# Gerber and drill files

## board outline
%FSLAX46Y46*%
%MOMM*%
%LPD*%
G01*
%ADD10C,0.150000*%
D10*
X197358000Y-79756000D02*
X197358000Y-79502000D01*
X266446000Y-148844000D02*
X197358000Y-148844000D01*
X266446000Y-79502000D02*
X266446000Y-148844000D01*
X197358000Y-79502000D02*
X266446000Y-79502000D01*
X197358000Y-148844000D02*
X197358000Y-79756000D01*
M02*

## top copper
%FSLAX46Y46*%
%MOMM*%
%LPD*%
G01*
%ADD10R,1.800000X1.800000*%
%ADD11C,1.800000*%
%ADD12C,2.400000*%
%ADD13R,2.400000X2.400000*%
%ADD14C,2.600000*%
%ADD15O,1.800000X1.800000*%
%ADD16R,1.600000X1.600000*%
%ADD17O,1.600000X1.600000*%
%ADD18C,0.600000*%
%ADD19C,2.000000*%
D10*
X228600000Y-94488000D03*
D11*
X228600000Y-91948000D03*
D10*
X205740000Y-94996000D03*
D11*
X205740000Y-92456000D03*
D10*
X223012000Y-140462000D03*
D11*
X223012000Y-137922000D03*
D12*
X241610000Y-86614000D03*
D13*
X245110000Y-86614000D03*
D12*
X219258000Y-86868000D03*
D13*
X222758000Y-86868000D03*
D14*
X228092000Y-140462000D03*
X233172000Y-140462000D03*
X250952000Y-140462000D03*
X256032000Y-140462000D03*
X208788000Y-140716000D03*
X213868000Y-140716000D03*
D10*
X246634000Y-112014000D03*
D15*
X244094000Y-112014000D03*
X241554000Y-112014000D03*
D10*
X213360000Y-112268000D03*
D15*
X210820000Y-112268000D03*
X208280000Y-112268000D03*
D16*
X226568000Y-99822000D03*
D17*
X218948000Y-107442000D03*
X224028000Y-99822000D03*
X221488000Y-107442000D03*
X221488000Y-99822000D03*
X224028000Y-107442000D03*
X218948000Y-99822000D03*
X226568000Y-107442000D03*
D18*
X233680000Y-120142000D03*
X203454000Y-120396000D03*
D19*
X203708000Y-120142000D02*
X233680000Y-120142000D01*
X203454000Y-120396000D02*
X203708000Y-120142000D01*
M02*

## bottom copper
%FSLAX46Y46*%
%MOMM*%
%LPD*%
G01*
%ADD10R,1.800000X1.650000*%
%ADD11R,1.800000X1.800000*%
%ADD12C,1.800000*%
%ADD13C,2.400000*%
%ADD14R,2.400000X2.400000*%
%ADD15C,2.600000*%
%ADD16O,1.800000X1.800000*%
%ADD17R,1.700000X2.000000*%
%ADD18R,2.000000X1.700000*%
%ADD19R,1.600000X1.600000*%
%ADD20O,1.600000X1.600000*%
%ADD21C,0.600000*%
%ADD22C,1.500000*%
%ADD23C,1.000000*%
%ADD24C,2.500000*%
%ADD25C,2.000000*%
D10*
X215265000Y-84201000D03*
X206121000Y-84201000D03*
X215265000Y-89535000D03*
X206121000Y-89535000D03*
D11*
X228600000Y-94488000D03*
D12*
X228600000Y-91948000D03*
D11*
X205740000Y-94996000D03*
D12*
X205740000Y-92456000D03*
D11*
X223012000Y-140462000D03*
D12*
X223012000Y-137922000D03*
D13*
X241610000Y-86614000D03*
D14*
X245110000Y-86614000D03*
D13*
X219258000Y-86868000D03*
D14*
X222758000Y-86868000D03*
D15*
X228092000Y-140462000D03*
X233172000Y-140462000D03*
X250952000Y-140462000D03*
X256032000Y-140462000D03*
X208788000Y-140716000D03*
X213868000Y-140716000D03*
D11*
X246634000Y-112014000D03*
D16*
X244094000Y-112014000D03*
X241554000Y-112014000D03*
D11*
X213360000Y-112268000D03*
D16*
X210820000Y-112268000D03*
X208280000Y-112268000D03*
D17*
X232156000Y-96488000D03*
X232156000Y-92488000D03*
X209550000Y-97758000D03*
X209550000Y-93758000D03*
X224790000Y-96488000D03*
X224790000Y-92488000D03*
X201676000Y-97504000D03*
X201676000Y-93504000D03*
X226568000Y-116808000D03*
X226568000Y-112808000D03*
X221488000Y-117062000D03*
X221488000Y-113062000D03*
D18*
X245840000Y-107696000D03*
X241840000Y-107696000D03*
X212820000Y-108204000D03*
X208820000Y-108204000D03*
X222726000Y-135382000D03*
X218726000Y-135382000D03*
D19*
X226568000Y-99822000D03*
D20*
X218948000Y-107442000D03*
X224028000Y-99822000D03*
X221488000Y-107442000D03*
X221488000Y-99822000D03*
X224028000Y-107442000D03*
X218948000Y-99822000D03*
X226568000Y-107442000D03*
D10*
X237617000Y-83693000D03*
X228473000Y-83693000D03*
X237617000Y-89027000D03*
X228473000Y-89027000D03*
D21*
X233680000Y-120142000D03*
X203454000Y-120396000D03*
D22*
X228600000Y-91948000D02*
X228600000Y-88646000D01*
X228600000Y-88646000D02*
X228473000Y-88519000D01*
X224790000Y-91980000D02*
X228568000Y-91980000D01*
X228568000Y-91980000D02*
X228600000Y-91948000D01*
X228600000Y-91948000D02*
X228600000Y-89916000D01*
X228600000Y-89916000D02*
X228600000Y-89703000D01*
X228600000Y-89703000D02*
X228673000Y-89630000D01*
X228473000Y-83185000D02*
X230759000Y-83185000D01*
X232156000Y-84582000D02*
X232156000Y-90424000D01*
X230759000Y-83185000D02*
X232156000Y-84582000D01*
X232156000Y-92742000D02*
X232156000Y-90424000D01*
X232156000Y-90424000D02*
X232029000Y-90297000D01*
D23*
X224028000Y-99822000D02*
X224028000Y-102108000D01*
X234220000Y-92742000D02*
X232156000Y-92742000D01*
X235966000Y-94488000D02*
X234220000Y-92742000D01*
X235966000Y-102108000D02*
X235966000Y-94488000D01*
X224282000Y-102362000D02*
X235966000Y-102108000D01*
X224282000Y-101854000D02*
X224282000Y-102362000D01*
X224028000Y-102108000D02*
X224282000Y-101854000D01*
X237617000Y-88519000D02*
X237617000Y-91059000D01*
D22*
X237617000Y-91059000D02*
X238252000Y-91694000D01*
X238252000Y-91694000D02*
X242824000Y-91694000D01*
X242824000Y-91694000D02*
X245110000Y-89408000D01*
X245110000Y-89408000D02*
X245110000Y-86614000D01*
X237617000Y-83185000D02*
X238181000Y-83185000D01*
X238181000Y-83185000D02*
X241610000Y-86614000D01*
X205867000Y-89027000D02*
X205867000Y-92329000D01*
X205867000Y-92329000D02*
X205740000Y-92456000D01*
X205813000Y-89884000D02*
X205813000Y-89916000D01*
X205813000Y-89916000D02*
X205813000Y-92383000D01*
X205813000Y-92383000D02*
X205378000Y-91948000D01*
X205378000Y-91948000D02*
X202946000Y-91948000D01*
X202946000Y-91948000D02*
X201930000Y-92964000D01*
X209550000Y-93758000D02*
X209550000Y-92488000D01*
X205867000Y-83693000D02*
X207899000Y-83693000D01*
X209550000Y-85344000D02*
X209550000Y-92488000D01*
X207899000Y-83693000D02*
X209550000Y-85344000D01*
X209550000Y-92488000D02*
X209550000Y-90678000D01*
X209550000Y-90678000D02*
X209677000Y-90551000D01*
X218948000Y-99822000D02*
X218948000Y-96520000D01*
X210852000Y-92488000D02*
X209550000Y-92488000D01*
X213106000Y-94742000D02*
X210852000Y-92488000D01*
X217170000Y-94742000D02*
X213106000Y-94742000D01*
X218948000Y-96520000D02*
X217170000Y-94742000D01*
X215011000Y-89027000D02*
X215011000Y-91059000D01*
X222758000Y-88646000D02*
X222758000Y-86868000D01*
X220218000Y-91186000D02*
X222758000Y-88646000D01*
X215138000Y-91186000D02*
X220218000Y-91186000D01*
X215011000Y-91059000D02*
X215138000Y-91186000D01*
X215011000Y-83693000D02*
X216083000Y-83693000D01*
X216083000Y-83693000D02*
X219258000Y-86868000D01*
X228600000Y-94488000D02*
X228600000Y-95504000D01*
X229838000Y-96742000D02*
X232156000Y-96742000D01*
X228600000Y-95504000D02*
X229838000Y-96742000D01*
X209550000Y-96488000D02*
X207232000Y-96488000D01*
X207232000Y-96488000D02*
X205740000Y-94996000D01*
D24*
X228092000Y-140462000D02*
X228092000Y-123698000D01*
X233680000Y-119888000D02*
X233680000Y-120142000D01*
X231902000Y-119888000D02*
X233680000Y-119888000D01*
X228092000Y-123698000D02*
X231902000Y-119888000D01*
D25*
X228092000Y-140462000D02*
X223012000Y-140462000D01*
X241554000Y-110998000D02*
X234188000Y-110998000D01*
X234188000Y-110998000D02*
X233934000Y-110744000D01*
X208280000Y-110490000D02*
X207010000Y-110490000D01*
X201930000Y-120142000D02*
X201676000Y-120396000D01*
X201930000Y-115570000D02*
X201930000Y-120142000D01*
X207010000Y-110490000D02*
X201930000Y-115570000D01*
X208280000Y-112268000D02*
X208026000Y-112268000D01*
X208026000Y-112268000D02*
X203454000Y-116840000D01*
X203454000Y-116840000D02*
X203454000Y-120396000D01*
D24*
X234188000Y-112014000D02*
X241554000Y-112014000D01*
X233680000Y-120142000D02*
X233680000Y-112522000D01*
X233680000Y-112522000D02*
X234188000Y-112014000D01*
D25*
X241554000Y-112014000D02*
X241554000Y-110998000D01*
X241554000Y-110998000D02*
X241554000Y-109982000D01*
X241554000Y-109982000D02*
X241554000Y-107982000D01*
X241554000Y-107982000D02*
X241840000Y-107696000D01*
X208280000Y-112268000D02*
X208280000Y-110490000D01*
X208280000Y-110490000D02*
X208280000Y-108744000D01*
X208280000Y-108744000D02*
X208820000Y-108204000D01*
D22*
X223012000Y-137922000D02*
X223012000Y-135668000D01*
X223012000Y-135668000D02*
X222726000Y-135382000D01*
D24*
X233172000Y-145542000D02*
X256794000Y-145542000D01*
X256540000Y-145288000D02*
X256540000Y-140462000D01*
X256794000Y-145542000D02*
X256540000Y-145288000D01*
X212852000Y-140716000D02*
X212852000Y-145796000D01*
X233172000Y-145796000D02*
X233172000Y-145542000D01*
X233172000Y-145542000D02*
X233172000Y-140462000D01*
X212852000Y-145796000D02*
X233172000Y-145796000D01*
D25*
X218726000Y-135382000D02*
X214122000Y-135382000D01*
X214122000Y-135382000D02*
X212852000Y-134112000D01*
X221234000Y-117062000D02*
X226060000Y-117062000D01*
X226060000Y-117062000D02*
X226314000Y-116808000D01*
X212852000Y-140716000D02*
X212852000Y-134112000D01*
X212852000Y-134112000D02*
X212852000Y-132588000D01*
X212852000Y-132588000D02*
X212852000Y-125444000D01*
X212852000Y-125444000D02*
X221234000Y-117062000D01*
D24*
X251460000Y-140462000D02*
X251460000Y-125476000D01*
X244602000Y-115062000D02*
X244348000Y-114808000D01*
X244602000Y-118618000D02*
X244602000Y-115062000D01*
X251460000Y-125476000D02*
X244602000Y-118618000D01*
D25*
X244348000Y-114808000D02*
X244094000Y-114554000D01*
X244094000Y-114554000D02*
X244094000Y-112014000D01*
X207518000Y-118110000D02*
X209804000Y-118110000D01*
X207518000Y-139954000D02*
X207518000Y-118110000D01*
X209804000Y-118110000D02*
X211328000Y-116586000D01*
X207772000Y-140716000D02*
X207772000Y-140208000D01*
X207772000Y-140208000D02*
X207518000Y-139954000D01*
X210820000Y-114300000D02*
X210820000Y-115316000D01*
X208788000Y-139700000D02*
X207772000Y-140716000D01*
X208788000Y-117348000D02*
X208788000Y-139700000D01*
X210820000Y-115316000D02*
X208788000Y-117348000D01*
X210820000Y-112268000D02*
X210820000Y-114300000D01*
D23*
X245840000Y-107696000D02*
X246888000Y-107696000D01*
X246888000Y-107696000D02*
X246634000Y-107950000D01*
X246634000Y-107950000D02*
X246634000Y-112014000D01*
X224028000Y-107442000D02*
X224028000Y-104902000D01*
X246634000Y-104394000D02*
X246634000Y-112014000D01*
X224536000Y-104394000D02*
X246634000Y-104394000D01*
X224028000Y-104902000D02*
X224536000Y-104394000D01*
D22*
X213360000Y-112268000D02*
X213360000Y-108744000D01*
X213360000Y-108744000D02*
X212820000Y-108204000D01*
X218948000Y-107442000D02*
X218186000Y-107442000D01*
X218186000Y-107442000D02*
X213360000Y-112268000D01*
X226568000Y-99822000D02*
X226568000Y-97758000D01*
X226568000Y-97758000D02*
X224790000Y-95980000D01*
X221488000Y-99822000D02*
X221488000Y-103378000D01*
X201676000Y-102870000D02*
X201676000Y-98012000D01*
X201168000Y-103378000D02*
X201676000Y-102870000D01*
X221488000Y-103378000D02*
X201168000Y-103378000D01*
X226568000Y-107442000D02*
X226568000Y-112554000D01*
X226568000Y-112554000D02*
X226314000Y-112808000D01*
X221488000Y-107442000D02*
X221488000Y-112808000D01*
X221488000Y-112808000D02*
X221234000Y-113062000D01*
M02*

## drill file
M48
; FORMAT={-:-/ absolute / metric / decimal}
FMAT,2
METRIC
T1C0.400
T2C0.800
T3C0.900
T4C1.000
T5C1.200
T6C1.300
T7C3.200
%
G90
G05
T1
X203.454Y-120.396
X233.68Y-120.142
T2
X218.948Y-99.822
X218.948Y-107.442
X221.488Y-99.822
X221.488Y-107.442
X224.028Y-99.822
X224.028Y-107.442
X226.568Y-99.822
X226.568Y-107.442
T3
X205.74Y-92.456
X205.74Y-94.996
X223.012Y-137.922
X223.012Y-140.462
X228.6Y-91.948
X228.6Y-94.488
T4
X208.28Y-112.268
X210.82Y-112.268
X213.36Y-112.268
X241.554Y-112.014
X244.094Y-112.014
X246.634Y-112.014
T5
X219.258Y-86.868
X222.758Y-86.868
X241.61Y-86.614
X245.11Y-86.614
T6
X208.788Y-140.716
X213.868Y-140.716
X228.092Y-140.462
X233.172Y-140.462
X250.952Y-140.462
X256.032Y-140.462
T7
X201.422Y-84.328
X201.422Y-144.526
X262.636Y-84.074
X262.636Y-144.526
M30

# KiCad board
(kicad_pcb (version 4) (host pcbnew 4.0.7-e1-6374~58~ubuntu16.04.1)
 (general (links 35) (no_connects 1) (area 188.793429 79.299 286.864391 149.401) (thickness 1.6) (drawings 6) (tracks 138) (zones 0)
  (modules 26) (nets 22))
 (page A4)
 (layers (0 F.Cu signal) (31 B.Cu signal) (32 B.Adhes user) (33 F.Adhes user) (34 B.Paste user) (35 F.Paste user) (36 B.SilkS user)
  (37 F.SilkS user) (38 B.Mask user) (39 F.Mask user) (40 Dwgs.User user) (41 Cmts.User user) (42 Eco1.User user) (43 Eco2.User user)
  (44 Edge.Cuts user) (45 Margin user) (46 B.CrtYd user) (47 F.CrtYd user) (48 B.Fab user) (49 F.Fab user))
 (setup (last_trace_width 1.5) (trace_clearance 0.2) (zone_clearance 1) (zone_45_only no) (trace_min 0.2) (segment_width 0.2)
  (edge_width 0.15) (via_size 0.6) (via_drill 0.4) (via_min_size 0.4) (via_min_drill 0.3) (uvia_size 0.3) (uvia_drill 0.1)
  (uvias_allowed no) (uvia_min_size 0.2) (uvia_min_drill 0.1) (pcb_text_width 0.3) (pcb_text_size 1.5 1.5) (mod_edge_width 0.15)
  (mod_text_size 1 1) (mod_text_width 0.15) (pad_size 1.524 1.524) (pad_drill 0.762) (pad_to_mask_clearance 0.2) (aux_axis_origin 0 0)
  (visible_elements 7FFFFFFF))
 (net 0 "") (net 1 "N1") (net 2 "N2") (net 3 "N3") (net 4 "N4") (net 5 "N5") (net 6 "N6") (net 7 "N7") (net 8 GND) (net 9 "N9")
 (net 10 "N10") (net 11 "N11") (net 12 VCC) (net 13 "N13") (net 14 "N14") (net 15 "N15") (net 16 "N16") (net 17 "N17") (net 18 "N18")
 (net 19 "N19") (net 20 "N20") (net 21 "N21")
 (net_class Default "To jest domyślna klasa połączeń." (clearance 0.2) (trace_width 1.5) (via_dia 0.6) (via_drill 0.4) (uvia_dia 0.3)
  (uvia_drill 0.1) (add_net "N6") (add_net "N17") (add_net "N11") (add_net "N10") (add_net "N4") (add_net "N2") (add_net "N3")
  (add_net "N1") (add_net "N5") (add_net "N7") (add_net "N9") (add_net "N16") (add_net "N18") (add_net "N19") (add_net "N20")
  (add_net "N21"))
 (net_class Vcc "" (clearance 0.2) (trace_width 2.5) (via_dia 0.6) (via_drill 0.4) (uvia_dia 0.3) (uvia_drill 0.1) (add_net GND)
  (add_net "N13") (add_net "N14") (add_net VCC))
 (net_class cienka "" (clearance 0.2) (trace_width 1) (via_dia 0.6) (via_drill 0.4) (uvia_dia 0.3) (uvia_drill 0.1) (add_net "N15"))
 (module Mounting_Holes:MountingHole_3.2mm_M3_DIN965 (layer F.Cu) (at 262.636 144.526)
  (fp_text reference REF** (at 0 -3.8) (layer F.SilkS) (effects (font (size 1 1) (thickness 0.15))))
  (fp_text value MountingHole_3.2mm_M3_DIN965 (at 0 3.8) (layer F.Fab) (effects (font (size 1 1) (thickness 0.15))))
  (pad 1 np_thru_hole circle (at 0 0) (size 3.2 3.2) (drill 3.2) (layers *.Cu *.Mask)))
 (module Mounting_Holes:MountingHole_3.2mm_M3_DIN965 (layer F.Cu) (at 201.422 144.526)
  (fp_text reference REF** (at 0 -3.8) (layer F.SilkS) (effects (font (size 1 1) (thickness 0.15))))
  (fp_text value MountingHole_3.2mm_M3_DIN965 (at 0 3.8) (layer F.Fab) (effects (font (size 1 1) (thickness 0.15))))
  (pad 1 np_thru_hole circle (at 0 0) (size 3.2 3.2) (drill 3.2) (layers *.Cu *.Mask)))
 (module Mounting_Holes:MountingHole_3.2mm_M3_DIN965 (layer F.Cu) (at 201.422 84.328)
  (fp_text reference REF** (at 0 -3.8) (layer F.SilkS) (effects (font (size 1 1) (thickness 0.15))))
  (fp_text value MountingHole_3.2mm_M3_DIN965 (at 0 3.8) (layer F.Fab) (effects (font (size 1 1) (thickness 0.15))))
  (pad 1 np_thru_hole circle (at 0 0) (size 3.2 3.2) (drill 3.2) (layers *.Cu *.Mask)))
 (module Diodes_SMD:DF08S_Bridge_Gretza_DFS (layer B.Cu) (at 210.566 86.868 270)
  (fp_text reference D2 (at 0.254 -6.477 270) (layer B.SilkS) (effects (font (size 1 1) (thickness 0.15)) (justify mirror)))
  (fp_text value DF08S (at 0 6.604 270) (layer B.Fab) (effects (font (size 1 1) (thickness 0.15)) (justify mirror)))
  (pad 4 smd rect (at -2.667 -4.699 270) (size 1.65 1.8) (layers B.Cu B.Paste B.Mask) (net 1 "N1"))
  (pad 2 smd rect (at -2.667 4.445 270) (size 1.65 1.8) (layers B.Cu B.Paste B.Mask) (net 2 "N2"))
  (pad 3 smd rect (at 2.667 -4.699 270) (size 1.65 1.8) (layers B.Cu B.Paste B.Mask) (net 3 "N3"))
  (pad 1 smd rect (at 2.667 4.445 270) (size 1.65 1.8) (layers B.Cu B.Paste B.Mask) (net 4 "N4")))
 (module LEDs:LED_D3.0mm (layer F.Cu) (at 228.6 94.488 90)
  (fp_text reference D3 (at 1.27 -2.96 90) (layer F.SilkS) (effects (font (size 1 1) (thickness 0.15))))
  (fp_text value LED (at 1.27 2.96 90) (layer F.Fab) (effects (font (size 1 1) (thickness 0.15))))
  (pad 1 thru_hole rect (at 0 0 90) (size 1.8 1.8) (drill 0.9) (layers *.Cu *.Mask) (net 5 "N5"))
  (pad 2 thru_hole circle (at 2.54 0 90) (size 1.8 1.8) (drill 0.9) (layers *.Cu *.Mask) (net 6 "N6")))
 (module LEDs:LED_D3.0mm (layer F.Cu) (at 205.74 94.996 90)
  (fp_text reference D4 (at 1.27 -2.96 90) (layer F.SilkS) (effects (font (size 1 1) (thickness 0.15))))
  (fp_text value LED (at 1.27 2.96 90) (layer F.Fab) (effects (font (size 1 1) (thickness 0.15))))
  (pad 1 thru_hole rect (at 0 0 90) (size 1.8 1.8) (drill 0.9) (layers *.Cu *.Mask) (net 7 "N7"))
  (pad 2 thru_hole circle (at 2.54 0 90) (size 1.8 1.8) (drill 0.9) (layers *.Cu *.Mask) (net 4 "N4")))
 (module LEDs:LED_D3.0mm (layer F.Cu) (at 223.012 140.462 90)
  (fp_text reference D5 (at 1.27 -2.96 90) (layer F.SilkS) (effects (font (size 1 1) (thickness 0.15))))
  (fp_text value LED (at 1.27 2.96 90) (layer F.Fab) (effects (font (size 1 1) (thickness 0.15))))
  (pad 1 thru_hole rect (at 0 0 90) (size 1.8 1.8) (drill 0.9) (layers *.Cu *.Mask) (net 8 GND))
  (pad 2 thru_hole circle (at 2.54 0 90) (size 1.8 1.8) (drill 0.9) (layers *.Cu *.Mask) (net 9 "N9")))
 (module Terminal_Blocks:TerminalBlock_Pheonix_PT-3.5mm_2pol (layer F.Cu) (at 245.11 86.614 180)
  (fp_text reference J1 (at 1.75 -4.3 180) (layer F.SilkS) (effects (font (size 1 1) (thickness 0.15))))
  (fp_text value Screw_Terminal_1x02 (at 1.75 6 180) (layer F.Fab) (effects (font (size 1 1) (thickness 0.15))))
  (pad 2 thru_hole circle (at 3.5 0 180) (size 2.4 2.4) (drill 1.2) (layers *.Cu *.Mask F.SilkS) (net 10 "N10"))
  (pad 1 thru_hole rect (at 0 0 180) (size 2.4 2.4) (drill 1.2) (layers *.Cu *.Mask F.SilkS) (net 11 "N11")))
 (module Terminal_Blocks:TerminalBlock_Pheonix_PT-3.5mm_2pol (layer F.Cu) (at 222.758 86.868 180)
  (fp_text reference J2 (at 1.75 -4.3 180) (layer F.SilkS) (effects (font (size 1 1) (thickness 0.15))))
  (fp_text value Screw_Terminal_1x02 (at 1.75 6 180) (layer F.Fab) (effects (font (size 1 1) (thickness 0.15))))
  (pad 2 thru_hole circle (at 3.5 0 180) (size 2.4 2.4) (drill 1.2) (layers *.Cu *.Mask F.SilkS) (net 1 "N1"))
  (pad 1 thru_hole rect (at 0 0 180) (size 2.4 2.4) (drill 1.2) (layers *.Cu *.Mask F.SilkS) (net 3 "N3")))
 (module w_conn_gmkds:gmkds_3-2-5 (layer F.Cu) (at 230.632 140.462)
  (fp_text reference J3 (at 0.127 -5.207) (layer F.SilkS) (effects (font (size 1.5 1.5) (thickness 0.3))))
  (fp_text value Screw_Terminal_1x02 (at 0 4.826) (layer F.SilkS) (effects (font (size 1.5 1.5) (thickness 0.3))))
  (pad 1 thru_hole circle (at -2.54 0) (size 2.6 2.6) (drill 1.3) (layers *.Cu *.Mask F.SilkS) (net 8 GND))
  (pad 2 thru_hole circle (at 2.54 0) (size 2.6 2.6) (drill 1.3) (layers *.Cu *.Mask F.SilkS) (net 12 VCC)))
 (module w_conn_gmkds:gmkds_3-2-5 (layer F.Cu) (at 253.492 140.462)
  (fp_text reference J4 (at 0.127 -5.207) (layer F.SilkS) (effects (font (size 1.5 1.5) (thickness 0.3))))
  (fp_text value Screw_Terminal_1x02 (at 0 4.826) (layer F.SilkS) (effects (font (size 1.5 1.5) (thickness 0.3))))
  (pad 1 thru_hole circle (at -2.54 0) (size 2.6 2.6) (drill 1.3) (layers *.Cu *.Mask F.SilkS) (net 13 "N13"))
  (pad 2 thru_hole circle (at 2.54 0) (size 2.6 2.6) (drill 1.3) (layers *.Cu *.Mask F.SilkS) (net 12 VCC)))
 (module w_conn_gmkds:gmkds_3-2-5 (layer F.Cu) (at 211.328 140.716)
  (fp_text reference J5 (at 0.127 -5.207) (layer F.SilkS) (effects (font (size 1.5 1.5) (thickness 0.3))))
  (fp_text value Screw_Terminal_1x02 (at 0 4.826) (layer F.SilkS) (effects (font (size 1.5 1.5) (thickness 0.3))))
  (pad 1 thru_hole circle (at -2.54 0) (size 2.6 2.6) (drill 1.3) (layers *.Cu *.Mask F.SilkS) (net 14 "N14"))
  (pad 2 thru_hole circle (at 2.54 0) (size 2.6 2.6) (drill 1.3) (layers *.Cu *.Mask F.SilkS) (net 12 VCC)))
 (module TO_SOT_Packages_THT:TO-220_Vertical (layer F.Cu) (at 246.634 112.014 180)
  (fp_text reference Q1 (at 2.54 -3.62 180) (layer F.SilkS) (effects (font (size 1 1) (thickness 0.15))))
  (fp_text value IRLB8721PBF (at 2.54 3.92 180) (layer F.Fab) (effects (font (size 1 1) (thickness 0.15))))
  (pad 1 thru_hole rect (at 0 0 180) (size 1.8 1.8) (drill 1) (layers *.Cu *.Mask) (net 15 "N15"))
  (pad 2 thru_hole oval (at 2.54 0 180) (size 1.8 1.8) (drill 1) (layers *.Cu *.Mask) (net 13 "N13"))
  (pad 3 thru_hole oval (at 5.08 0 180) (size 1.8 1.8) (drill 1) (layers *.Cu *.Mask) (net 8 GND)))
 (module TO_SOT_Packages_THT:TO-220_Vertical (layer F.Cu) (at 213.36 112.268 180)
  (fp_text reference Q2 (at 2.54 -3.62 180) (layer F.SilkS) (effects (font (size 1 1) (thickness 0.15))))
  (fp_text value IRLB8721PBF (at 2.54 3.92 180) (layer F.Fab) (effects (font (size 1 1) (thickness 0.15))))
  (pad 1 thru_hole rect (at 0 0 180) (size 1.8 1.8) (drill 1) (layers *.Cu *.Mask) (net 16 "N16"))
  (pad 2 thru_hole oval (at 2.54 0 180) (size 1.8 1.8) (drill 1) (layers *.Cu *.Mask) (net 14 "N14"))
  (pad 3 thru_hole oval (at 5.08 0 180) (size 1.8 1.8) (drill 1) (layers *.Cu *.Mask) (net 8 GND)))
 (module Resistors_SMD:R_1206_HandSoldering (layer B.Cu) (at 232.156 94.488 90)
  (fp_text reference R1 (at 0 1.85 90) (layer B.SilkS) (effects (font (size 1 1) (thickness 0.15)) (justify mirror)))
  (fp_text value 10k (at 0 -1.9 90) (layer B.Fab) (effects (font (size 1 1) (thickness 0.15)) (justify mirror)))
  (pad 1 smd rect (at -2 0 90) (size 2 1.7) (layers B.Cu B.Paste B.Mask) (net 5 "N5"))
  (pad 2 smd rect (at 2 0 90) (size 2 1.7) (layers B.Cu B.Paste B.Mask) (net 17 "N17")))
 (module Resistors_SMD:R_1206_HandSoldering (layer B.Cu) (at 209.55 95.758 90)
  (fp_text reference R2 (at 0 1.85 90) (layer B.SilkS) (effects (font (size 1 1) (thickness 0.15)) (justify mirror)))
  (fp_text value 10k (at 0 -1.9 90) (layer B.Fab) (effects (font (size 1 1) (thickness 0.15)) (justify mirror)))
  (pad 1 smd rect (at -2 0 90) (size 2 1.7) (layers B.Cu B.Paste B.Mask) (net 7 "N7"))
  (pad 2 smd rect (at 2 0 90) (size 2 1.7) (layers B.Cu B.Paste B.Mask) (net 2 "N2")))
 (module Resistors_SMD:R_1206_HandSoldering (layer B.Cu) (at 224.79 94.488 90)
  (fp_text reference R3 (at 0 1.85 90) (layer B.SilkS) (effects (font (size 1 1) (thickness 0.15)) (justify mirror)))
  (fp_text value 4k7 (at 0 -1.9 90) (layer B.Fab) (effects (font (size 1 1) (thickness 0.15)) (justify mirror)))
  (pad 1 smd rect (at -2 0 90) (size 2 1.7) (layers B.Cu B.Paste B.Mask) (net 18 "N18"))
  (pad 2 smd rect (at 2 0 90) (size 2 1.7) (layers B.Cu B.Paste B.Mask) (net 6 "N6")))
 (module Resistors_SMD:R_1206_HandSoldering (layer B.Cu) (at 201.676 95.504 90)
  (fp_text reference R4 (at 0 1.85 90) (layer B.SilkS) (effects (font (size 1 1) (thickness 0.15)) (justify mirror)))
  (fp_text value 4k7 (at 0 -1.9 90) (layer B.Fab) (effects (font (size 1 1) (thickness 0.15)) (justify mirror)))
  (pad 1 smd rect (at -2 0 90) (size 2 1.7) (layers B.Cu B.Paste B.Mask) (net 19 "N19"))
  (pad 2 smd rect (at 2 0 90) (size 2 1.7) (layers B.Cu B.Paste B.Mask) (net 4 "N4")))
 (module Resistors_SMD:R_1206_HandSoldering (layer B.Cu) (at 226.568 114.808 90)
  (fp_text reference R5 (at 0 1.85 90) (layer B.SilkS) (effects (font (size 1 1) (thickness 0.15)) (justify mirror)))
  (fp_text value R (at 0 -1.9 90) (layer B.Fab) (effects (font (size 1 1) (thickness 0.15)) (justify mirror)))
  (pad 1 smd rect (at -2 0 90) (size 2 1.7) (layers B.Cu B.Paste B.Mask) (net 12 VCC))
  (pad 2 smd rect (at 2 0 90) (size 2 1.7) (layers B.Cu B.Paste B.Mask) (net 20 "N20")))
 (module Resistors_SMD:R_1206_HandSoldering (layer B.Cu) (at 221.488 115.062 90)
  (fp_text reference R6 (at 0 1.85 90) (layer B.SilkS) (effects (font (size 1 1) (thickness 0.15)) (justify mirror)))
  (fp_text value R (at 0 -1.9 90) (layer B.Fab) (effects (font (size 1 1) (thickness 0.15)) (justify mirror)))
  (pad 1 smd rect (at -2 0 90) (size 2 1.7) (layers B.Cu B.Paste B.Mask) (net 12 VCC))
  (pad 2 smd rect (at 2 0 90) (size 2 1.7) (layers B.Cu B.Paste B.Mask) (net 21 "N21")))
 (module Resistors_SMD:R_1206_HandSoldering (layer B.Cu) (at 243.84 107.696 180)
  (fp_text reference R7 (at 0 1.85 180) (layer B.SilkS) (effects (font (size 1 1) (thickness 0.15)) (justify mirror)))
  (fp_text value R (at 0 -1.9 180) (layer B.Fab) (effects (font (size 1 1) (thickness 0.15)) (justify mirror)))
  (pad 1 smd rect (at -2 0 180) (size 2 1.7) (layers B.Cu B.Paste B.Mask) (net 15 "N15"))
  (pad 2 smd rect (at 2 0 180) (size 2 1.7) (layers B.Cu B.Paste B.Mask) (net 8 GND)))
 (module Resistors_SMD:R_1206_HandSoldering (layer B.Cu) (at 210.82 108.204 180)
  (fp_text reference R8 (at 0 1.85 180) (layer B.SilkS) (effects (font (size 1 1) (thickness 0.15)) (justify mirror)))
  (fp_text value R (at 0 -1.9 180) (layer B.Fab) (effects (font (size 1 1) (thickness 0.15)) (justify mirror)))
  (pad 1 smd rect (at -2 0 180) (size 2 1.7) (layers B.Cu B.Paste B.Mask) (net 16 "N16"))
  (pad 2 smd rect (at 2 0 180) (size 2 1.7) (layers B.Cu B.Paste B.Mask) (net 8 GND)))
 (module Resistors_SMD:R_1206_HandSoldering (layer B.Cu) (at 220.726 135.382 180)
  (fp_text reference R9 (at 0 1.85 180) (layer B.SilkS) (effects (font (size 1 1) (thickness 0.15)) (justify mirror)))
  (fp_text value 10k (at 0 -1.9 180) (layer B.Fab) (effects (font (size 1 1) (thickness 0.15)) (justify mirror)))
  (pad 1 smd rect (at -2 0 180) (size 2 1.7) (layers B.Cu B.Paste B.Mask) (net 9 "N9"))
  (pad 2 smd rect (at 2 0 180) (size 2 1.7) (layers B.Cu B.Paste B.Mask) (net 12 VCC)))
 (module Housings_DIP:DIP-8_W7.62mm (layer F.Cu) (at 226.568 99.822 270)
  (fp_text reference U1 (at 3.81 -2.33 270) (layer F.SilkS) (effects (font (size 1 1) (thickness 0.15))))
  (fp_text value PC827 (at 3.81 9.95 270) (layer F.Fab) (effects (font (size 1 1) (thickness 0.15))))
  (pad 1 thru_hole rect (at 0 0 270) (size 1.6 1.6) (drill 0.8) (layers *.Cu *.Mask) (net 18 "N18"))
  (pad 5 thru_hole oval (at 7.62 7.62 270) (size 1.6 1.6) (drill 0.8) (layers *.Cu *.Mask) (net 16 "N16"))
  (pad 2 thru_hole oval (at 0 2.54 270) (size 1.6 1.6) (drill 0.8) (layers *.Cu *.Mask) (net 17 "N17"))
  (pad 6 thru_hole oval (at 7.62 5.08 270) (size 1.6 1.6) (drill 0.8) (layers *.Cu *.Mask) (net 21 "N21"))
  (pad 3 thru_hole oval (at 0 5.08 270) (size 1.6 1.6) (drill 0.8) (layers *.Cu *.Mask) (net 19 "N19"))
  (pad 7 thru_hole oval (at 7.62 2.54 270) (size 1.6 1.6) (drill 0.8) (layers *.Cu *.Mask) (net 15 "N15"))
  (pad 4 thru_hole oval (at 0 7.62 270) (size 1.6 1.6) (drill 0.8) (layers *.Cu *.Mask) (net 2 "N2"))
  (pad 8 thru_hole oval (at 7.62 0 270) (size 1.6 1.6) (drill 0.8) (layers *.Cu *.Mask) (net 20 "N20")))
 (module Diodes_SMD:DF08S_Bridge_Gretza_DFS (layer B.Cu) (at 232.918 86.36 270)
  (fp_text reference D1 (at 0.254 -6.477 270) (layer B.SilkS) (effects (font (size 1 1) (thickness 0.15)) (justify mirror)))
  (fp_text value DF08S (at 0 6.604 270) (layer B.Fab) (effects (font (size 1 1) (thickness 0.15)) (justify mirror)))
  (pad 4 smd rect (at -2.667 -4.699 270) (size 1.65 1.8) (layers B.Cu B.Paste B.Mask) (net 10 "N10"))
  (pad 2 smd rect (at -2.667 4.445 270) (size 1.65 1.8) (layers B.Cu B.Paste B.Mask) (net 17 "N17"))
  (pad 3 smd rect (at 2.667 -4.699 270) (size 1.65 1.8) (layers B.Cu B.Paste B.Mask) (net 11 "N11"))
  (pad 1 smd rect (at 2.667 4.445 270) (size 1.65 1.8) (layers B.Cu B.Paste B.Mask) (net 6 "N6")))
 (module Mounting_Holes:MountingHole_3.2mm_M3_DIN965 (layer F.Cu) (at 262.636 84.074)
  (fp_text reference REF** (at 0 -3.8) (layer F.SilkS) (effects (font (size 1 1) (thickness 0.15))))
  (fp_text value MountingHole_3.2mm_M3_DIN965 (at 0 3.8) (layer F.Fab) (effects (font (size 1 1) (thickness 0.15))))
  (pad 1 np_thru_hole circle (at 0 0) (size 3.2 3.2) (drill 3.2) (layers *.Cu *.Mask)))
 (gr_line (start 197.358 79.756) (end 197.358 79.502) (angle 90) (layer Edge.Cuts) (width 0.15))
 (gr_line (start 266.446 148.844) (end 197.358 148.844) (angle 90) (layer Edge.Cuts) (width 0.15))
 (gr_line (start 266.446 79.502) (end 266.446 148.844) (angle 90) (layer Edge.Cuts) (width 0.15))
 (gr_line (start 197.358 79.502) (end 266.446 79.502) (angle 90) (layer Edge.Cuts) (width 0.15))
 (gr_line (start 197.358 148.844) (end 197.358 79.756) (angle 90) (layer Edge.Cuts) (width 0.15))
 (segment (start 228.6 91.948) (end 228.6 88.646) (width 1.5) (layer B.Cu) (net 6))
 (segment (start 228.6 88.646) (end 228.473 88.519) (width 1.5) (layer B.Cu) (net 6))
 (segment (start 224.79 91.98) (end 228.568 91.98) (width 1.5) (layer B.Cu) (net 6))
 (segment (start 228.568 91.98) (end 228.6 91.948) (width 1.5) (layer B.Cu) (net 6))
 (segment (start 228.6 91.948) (end 228.6 89.916) (width 1.5) (layer B.Cu) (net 6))
 (segment (start 228.6 89.916) (end 228.6 89.703) (width 1.5) (layer B.Cu) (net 6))
 (segment (start 228.6 89.703) (end 228.673 89.63) (width 1.5) (layer B.Cu) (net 6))
 (segment (start 228.473 83.185) (end 230.759 83.185) (width 1.5) (layer B.Cu) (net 17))
 (segment (start 232.156 84.582) (end 232.156 90.424) (width 1.5) (layer B.Cu) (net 17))
 (segment (start 230.759 83.185) (end 232.156 84.582) (width 1.5) (layer B.Cu) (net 17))
 (segment (start 232.156 92.742) (end 232.156 90.424) (width 1.5) (layer B.Cu) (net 17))
 (segment (start 232.156 90.424) (end 232.029 90.297) (width 1.5) (layer B.Cu) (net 17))
 (segment (start 224.028 99.822) (end 224.028 102.108) (width 1) (layer B.Cu) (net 17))
 (segment (start 234.22 92.742) (end 232.156 92.742) (width 1) (layer B.Cu) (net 17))
 (segment (start 235.966 94.488) (end 234.22 92.742) (width 1) (layer B.Cu) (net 17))
 (segment (start 235.966 102.108) (end 235.966 94.488) (width 1) (layer B.Cu) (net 17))
 (segment (start 224.282 102.362) (end 235.966 102.108) (width 1) (layer B.Cu) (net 17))
 (segment (start 224.282 101.854) (end 224.282 102.362) (width 1) (layer B.Cu) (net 17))
 (segment (start 224.028 102.108) (end 224.282 101.854) (width 1) (layer B.Cu) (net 17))
 (segment (start 237.617 88.519) (end 237.617 91.059) (width 1) (layer B.Cu) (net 11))
 (segment (start 237.617 91.059) (end 238.252 91.694) (width 1.5) (layer B.Cu) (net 11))
 (segment (start 238.252 91.694) (end 242.824 91.694) (width 1.5) (layer B.Cu) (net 11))
 (segment (start 242.824 91.694) (end 245.11 89.408) (width 1.5) (layer B.Cu) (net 11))
 (segment (start 245.11 89.408) (end 245.11 86.614) (width 1.5) (layer B.Cu) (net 11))
 (segment (start 237.617 83.185) (end 238.181 83.185) (width 1.5) (layer B.Cu) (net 10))
 (segment (start 238.181 83.185) (end 241.61 86.614) (width 1.5) (layer B.Cu) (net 10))
 (segment (start 205.867 89.027) (end 205.867 92.329) (width 1.5) (layer B.Cu) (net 4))
 (segment (start 205.867 92.329) (end 205.74 92.456) (width 1.5) (layer B.Cu) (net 4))
 (segment (start 205.813 89.884) (end 205.813 89.916) (width 1.5) (layer B.Cu) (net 4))
 (segment (start 205.813 89.916) (end 205.813 92.383) (width 1.5) (layer B.Cu) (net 4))
 (segment (start 205.813 92.383) (end 205.378 91.948) (width 1.5) (layer B.Cu) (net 4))
 (segment (start 205.378 91.948) (end 202.946 91.948) (width 1.5) (layer B.Cu) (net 4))
 (segment (start 202.946 91.948) (end 201.93 92.964) (width 1.5) (layer B.Cu) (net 4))
 (segment (start 209.55 93.758) (end 209.55 92.488) (width 1.5) (layer B.Cu) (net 2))
 (segment (start 205.867 83.693) (end 207.899 83.693) (width 1.5) (layer B.Cu) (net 2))
 (segment (start 209.55 85.344) (end 209.55 92.488) (width 1.5) (layer B.Cu) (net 2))
 (segment (start 207.899 83.693) (end 209.55 85.344) (width 1.5) (layer B.Cu) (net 2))
 (segment (start 209.55 92.488) (end 209.55 90.678) (width 1.5) (layer B.Cu) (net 2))
 (segment (start 209.55 90.678) (end 209.677 90.551) (width 1.5) (layer B.Cu) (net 2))
 (segment (start 218.948 99.822) (end 218.948 96.52) (width 1.5) (layer B.Cu) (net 2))
 (segment (start 210.852 92.488) (end 209.55 92.488) (width 1.5) (layer B.Cu) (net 2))
 (segment (start 213.106 94.742) (end 210.852 92.488) (width 1.5) (layer B.Cu) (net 2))
 (segment (start 217.17 94.742) (end 213.106 94.742) (width 1.5) (layer B.Cu) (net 2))
 (segment (start 218.948 96.52) (end 217.17 94.742) (width 1.5) (layer B.Cu) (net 2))
 (segment (start 215.011 89.027) (end 215.011 91.059) (width 1.5) (layer B.Cu) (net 3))
 (segment (start 222.758 88.646) (end 222.758 86.868) (width 1.5) (layer B.Cu) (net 3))
 (segment (start 220.218 91.186) (end 222.758 88.646) (width 1.5) (layer B.Cu) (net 3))
 (segment (start 215.138 91.186) (end 220.218 91.186) (width 1.5) (layer B.Cu) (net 3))
 (segment (start 215.011 91.059) (end 215.138 91.186) (width 1.5) (layer B.Cu) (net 3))
 (segment (start 215.011 83.693) (end 216.083 83.693) (width 1.5) (layer B.Cu) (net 1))
 (segment (start 216.083 83.693) (end 219.258 86.868) (width 1.5) (layer B.Cu) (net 1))
 (segment (start 228.6 94.488) (end 228.6 95.504) (width 1.5) (layer B.Cu) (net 5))
 (segment (start 229.838 96.742) (end 232.156 96.742) (width 1.5) (layer B.Cu) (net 5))
 (segment (start 228.6 95.504) (end 229.838 96.742) (width 1.5) (layer B.Cu) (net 5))
 (segment (start 209.55 96.488) (end 207.232 96.488) (width 1.5) (layer B.Cu) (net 7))
 (segment (start 207.232 96.488) (end 205.74 94.996) (width 1.5) (layer B.Cu) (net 7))
 (segment (start 228.092 140.462) (end 228.092 123.698) (width 2.5) (layer B.Cu) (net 8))
 (segment (start 233.68 119.888) (end 233.68 120.142) (width 2.5) (layer B.Cu) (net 8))
 (segment (start 231.902 119.888) (end 233.68 119.888) (width 2.5) (layer B.Cu) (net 8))
 (segment (start 228.092 123.698) (end 231.902 119.888) (width 2.5) (layer B.Cu) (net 8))
 (segment (start 228.092 140.462) (end 223.012 140.462) (width 2) (layer B.Cu) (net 8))
 (segment (start 241.554 110.998) (end 234.188 110.998) (width 2) (layer B.Cu) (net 8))
 (segment (start 234.188 110.998) (end 233.934 110.744) (width 2) (layer B.Cu) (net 8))
 (segment (start 208.28 110.49) (end 207.01 110.49) (width 2) (layer B.Cu) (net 8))
 (segment (start 201.93 120.142) (end 201.676 120.396) (width 2) (layer B.Cu) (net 8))
 (segment (start 201.93 115.57) (end 201.93 120.142) (width 2) (layer B.Cu) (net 8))
 (segment (start 207.01 110.49) (end 201.93 115.57) (width 2) (layer B.Cu) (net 8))
 (segment (start 208.28 112.268) (end 208.026 112.268) (width 2) (layer B.Cu) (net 8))
 (segment (start 208.026 112.268) (end 203.454 116.84) (width 2) (layer B.Cu) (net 8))
 (via (at 233.68 120.142) (size 0.6) (drill 0.4) (layers F.Cu B.Cu) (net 8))
 (segment (start 203.708 120.142) (end 233.68 120.142) (width 2) (layer F.Cu) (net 8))
 (segment (start 203.454 120.396) (end 203.708 120.142) (width 2) (layer F.Cu) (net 8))
 (via (at 203.454 120.396) (size 0.6) (drill 0.4) (layers F.Cu B.Cu) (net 8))
 (segment (start 203.454 116.84) (end 203.454 120.396) (width 2) (layer B.Cu) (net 8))
 (segment (start 234.188 112.014) (end 241.554 112.014) (width 2.5) (layer B.Cu) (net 8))
 (segment (start 233.68 120.142) (end 233.68 112.522) (width 2.5) (layer B.Cu) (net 8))
 (segment (start 233.68 112.522) (end 234.188 112.014) (width 2.5) (layer B.Cu) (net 8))
 (segment (start 241.554 112.014) (end 241.554 110.998) (width 2) (layer B.Cu) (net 8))
 (segment (start 241.554 110.998) (end 241.554 109.982) (width 2) (layer B.Cu) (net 8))
 (segment (start 241.554 109.982) (end 241.554 107.982) (width 2) (layer B.Cu) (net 8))
 (segment (start 241.554 107.982) (end 241.84 107.696) (width 2) (layer B.Cu) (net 8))
 (segment (start 208.28 112.268) (end 208.28 110.49) (width 2) (layer B.Cu) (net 8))
 (segment (start 208.28 110.49) (end 208.28 108.744) (width 2) (layer B.Cu) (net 8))
 (segment (start 208.28 108.744) (end 208.82 108.204) (width 2) (layer B.Cu) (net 8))
 (segment (start 223.012 137.922) (end 223.012 135.668) (width 1.5) (layer B.Cu) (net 9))
 (segment (start 223.012 135.668) (end 222.726 135.382) (width 1.5) (layer B.Cu) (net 9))
 (segment (start 233.172 145.542) (end 256.794 145.542) (width 2.5) (layer B.Cu) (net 12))
 (segment (start 256.54 145.288) (end 256.54 140.462) (width 2.5) (layer B.Cu) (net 12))
 (segment (start 256.794 145.542) (end 256.54 145.288) (width 2.5) (layer B.Cu) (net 12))
 (segment (start 212.852 140.716) (end 212.852 145.796) (width 2.5) (layer B.Cu) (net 12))
 (segment (start 233.172 145.796) (end 233.172 145.542) (width 2.5) (layer B.Cu) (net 12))
 (segment (start 233.172 145.542) (end 233.172 140.462) (width 2.5) (layer B.Cu) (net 12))
 (segment (start 212.852 145.796) (end 233.172 145.796) (width 2.5) (layer B.Cu) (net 12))
 (segment (start 218.726 135.382) (end 214.122 135.382) (width 2) (layer B.Cu) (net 12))
 (segment (start 214.122 135.382) (end 212.852 134.112) (width 2) (layer B.Cu) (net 12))
 (segment (start 221.234 117.062) (end 226.06 117.062) (width 2) (layer B.Cu) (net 12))
 (segment (start 226.06 117.062) (end 226.314 116.808) (width 2) (layer B.Cu) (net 12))
 (segment (start 212.852 140.716) (end 212.852 134.112) (width 2) (layer B.Cu) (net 12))
 (segment (start 212.852 134.112) (end 212.852 132.588) (width 2) (layer B.Cu) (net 12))
 (segment (start 212.852 132.588) (end 212.852 125.444) (width 2) (layer B.Cu) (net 12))
 (segment (start 212.852 125.444) (end 221.234 117.062) (width 2) (layer B.Cu) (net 12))
 (segment (start 251.46 140.462) (end 251.46 125.476) (width 2.5) (layer B.Cu) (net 13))
 (segment (start 244.602 115.062) (end 244.348 114.808) (width 2.5) (layer B.Cu) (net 13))
 (segment (start 244.602 118.618) (end 244.602 115.062) (width 2.5) (layer B.Cu) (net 13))
 (segment (start 251.46 125.476) (end 244.602 118.618) (width 2.5) (layer B.Cu) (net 13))
 (segment (start 244.348 114.808) (end 244.094 114.554) (width 2) (layer B.Cu) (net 13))
 (segment (start 244.094 114.554) (end 244.094 112.014) (width 2) (layer B.Cu) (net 13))
 (segment (start 207.518 118.11) (end 209.804 118.11) (width 2) (layer B.Cu) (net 14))
 (segment (start 207.518 139.954) (end 207.518 118.11) (width 2) (layer B.Cu) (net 14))
 (segment (start 209.804 118.11) (end 211.328 116.586) (width 2) (layer B.Cu) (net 14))
 (segment (start 207.772 140.716) (end 207.772 140.208) (width 2) (layer B.Cu) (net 14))
 (segment (start 207.772 140.208) (end 207.518 139.954) (width 2) (layer B.Cu) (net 14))
 (segment (start 210.82 114.3) (end 210.82 115.316) (width 2) (layer B.Cu) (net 14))
 (segment (start 208.788 139.7) (end 207.772 140.716) (width 2) (layer B.Cu) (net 14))
 (segment (start 208.788 117.348) (end 208.788 139.7) (width 2) (layer B.Cu) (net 14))
 (segment (start 210.82 115.316) (end 208.788 117.348) (width 2) (layer B.Cu) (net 14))
 (segment (start 210.82 112.268) (end 210.82 114.3) (width 2) (layer B.Cu) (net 14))
 (segment (start 245.84 107.696) (end 246.888 107.696) (width 1) (layer B.Cu) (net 15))
 (segment (start 246.888 107.696) (end 246.634 107.95) (width 1) (layer B.Cu) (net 15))
 (segment (start 246.634 107.95) (end 246.634 112.014) (width 1) (layer B.Cu) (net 15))
 (segment (start 224.028 107.442) (end 224.028 104.902) (width 1) (layer B.Cu) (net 15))
 (segment (start 246.634 104.394) (end 246.634 112.014) (width 1) (layer B.Cu) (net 15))
 (segment (start 224.536 104.394) (end 246.634 104.394) (width 1) (layer B.Cu) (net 15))
 (segment (start 224.028 104.902) (end 224.536 104.394) (width 1) (layer B.Cu) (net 15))
 (segment (start 213.36 112.268) (end 213.36 108.744) (width 1.5) (layer B.Cu) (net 16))
 (segment (start 213.36 108.744) (end 212.82 108.204) (width 1.5) (layer B.Cu) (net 16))
 (segment (start 218.948 107.442) (end 218.186 107.442) (width 1.5) (layer B.Cu) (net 16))
 (segment (start 218.186 107.442) (end 213.36 112.268) (width 1.5) (layer B.Cu) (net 16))
 (segment (start 226.568 99.822) (end 226.568 97.758) (width 1.5) (layer B.Cu) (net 18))
 (segment (start 226.568 97.758) (end 224.79 95.98) (width 1.5) (layer B.Cu) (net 18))
 (segment (start 221.488 99.822) (end 221.488 103.378) (width 1.5) (layer B.Cu) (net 19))
 (segment (start 201.676 102.87) (end 201.676 98.012) (width 1.5) (layer B.Cu) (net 19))
 (segment (start 201.168 103.378) (end 201.676 102.87) (width 1.5) (layer B.Cu) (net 19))
 (segment (start 221.488 103.378) (end 201.168 103.378) (width 1.5) (layer B.Cu) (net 19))
 (segment (start 226.568 107.442) (end 226.568 112.554) (width 1.5) (layer B.Cu) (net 20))
 (segment (start 226.568 112.554) (end 226.314 112.808) (width 1.5) (layer B.Cu) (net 20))
 (segment (start 221.488 107.442) (end 221.488 112.808) (width 1.5) (layer B.Cu) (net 21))
 (segment (start 221.488 112.808) (end 221.234 113.062) (width 1.5) (layer B.Cu) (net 21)))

